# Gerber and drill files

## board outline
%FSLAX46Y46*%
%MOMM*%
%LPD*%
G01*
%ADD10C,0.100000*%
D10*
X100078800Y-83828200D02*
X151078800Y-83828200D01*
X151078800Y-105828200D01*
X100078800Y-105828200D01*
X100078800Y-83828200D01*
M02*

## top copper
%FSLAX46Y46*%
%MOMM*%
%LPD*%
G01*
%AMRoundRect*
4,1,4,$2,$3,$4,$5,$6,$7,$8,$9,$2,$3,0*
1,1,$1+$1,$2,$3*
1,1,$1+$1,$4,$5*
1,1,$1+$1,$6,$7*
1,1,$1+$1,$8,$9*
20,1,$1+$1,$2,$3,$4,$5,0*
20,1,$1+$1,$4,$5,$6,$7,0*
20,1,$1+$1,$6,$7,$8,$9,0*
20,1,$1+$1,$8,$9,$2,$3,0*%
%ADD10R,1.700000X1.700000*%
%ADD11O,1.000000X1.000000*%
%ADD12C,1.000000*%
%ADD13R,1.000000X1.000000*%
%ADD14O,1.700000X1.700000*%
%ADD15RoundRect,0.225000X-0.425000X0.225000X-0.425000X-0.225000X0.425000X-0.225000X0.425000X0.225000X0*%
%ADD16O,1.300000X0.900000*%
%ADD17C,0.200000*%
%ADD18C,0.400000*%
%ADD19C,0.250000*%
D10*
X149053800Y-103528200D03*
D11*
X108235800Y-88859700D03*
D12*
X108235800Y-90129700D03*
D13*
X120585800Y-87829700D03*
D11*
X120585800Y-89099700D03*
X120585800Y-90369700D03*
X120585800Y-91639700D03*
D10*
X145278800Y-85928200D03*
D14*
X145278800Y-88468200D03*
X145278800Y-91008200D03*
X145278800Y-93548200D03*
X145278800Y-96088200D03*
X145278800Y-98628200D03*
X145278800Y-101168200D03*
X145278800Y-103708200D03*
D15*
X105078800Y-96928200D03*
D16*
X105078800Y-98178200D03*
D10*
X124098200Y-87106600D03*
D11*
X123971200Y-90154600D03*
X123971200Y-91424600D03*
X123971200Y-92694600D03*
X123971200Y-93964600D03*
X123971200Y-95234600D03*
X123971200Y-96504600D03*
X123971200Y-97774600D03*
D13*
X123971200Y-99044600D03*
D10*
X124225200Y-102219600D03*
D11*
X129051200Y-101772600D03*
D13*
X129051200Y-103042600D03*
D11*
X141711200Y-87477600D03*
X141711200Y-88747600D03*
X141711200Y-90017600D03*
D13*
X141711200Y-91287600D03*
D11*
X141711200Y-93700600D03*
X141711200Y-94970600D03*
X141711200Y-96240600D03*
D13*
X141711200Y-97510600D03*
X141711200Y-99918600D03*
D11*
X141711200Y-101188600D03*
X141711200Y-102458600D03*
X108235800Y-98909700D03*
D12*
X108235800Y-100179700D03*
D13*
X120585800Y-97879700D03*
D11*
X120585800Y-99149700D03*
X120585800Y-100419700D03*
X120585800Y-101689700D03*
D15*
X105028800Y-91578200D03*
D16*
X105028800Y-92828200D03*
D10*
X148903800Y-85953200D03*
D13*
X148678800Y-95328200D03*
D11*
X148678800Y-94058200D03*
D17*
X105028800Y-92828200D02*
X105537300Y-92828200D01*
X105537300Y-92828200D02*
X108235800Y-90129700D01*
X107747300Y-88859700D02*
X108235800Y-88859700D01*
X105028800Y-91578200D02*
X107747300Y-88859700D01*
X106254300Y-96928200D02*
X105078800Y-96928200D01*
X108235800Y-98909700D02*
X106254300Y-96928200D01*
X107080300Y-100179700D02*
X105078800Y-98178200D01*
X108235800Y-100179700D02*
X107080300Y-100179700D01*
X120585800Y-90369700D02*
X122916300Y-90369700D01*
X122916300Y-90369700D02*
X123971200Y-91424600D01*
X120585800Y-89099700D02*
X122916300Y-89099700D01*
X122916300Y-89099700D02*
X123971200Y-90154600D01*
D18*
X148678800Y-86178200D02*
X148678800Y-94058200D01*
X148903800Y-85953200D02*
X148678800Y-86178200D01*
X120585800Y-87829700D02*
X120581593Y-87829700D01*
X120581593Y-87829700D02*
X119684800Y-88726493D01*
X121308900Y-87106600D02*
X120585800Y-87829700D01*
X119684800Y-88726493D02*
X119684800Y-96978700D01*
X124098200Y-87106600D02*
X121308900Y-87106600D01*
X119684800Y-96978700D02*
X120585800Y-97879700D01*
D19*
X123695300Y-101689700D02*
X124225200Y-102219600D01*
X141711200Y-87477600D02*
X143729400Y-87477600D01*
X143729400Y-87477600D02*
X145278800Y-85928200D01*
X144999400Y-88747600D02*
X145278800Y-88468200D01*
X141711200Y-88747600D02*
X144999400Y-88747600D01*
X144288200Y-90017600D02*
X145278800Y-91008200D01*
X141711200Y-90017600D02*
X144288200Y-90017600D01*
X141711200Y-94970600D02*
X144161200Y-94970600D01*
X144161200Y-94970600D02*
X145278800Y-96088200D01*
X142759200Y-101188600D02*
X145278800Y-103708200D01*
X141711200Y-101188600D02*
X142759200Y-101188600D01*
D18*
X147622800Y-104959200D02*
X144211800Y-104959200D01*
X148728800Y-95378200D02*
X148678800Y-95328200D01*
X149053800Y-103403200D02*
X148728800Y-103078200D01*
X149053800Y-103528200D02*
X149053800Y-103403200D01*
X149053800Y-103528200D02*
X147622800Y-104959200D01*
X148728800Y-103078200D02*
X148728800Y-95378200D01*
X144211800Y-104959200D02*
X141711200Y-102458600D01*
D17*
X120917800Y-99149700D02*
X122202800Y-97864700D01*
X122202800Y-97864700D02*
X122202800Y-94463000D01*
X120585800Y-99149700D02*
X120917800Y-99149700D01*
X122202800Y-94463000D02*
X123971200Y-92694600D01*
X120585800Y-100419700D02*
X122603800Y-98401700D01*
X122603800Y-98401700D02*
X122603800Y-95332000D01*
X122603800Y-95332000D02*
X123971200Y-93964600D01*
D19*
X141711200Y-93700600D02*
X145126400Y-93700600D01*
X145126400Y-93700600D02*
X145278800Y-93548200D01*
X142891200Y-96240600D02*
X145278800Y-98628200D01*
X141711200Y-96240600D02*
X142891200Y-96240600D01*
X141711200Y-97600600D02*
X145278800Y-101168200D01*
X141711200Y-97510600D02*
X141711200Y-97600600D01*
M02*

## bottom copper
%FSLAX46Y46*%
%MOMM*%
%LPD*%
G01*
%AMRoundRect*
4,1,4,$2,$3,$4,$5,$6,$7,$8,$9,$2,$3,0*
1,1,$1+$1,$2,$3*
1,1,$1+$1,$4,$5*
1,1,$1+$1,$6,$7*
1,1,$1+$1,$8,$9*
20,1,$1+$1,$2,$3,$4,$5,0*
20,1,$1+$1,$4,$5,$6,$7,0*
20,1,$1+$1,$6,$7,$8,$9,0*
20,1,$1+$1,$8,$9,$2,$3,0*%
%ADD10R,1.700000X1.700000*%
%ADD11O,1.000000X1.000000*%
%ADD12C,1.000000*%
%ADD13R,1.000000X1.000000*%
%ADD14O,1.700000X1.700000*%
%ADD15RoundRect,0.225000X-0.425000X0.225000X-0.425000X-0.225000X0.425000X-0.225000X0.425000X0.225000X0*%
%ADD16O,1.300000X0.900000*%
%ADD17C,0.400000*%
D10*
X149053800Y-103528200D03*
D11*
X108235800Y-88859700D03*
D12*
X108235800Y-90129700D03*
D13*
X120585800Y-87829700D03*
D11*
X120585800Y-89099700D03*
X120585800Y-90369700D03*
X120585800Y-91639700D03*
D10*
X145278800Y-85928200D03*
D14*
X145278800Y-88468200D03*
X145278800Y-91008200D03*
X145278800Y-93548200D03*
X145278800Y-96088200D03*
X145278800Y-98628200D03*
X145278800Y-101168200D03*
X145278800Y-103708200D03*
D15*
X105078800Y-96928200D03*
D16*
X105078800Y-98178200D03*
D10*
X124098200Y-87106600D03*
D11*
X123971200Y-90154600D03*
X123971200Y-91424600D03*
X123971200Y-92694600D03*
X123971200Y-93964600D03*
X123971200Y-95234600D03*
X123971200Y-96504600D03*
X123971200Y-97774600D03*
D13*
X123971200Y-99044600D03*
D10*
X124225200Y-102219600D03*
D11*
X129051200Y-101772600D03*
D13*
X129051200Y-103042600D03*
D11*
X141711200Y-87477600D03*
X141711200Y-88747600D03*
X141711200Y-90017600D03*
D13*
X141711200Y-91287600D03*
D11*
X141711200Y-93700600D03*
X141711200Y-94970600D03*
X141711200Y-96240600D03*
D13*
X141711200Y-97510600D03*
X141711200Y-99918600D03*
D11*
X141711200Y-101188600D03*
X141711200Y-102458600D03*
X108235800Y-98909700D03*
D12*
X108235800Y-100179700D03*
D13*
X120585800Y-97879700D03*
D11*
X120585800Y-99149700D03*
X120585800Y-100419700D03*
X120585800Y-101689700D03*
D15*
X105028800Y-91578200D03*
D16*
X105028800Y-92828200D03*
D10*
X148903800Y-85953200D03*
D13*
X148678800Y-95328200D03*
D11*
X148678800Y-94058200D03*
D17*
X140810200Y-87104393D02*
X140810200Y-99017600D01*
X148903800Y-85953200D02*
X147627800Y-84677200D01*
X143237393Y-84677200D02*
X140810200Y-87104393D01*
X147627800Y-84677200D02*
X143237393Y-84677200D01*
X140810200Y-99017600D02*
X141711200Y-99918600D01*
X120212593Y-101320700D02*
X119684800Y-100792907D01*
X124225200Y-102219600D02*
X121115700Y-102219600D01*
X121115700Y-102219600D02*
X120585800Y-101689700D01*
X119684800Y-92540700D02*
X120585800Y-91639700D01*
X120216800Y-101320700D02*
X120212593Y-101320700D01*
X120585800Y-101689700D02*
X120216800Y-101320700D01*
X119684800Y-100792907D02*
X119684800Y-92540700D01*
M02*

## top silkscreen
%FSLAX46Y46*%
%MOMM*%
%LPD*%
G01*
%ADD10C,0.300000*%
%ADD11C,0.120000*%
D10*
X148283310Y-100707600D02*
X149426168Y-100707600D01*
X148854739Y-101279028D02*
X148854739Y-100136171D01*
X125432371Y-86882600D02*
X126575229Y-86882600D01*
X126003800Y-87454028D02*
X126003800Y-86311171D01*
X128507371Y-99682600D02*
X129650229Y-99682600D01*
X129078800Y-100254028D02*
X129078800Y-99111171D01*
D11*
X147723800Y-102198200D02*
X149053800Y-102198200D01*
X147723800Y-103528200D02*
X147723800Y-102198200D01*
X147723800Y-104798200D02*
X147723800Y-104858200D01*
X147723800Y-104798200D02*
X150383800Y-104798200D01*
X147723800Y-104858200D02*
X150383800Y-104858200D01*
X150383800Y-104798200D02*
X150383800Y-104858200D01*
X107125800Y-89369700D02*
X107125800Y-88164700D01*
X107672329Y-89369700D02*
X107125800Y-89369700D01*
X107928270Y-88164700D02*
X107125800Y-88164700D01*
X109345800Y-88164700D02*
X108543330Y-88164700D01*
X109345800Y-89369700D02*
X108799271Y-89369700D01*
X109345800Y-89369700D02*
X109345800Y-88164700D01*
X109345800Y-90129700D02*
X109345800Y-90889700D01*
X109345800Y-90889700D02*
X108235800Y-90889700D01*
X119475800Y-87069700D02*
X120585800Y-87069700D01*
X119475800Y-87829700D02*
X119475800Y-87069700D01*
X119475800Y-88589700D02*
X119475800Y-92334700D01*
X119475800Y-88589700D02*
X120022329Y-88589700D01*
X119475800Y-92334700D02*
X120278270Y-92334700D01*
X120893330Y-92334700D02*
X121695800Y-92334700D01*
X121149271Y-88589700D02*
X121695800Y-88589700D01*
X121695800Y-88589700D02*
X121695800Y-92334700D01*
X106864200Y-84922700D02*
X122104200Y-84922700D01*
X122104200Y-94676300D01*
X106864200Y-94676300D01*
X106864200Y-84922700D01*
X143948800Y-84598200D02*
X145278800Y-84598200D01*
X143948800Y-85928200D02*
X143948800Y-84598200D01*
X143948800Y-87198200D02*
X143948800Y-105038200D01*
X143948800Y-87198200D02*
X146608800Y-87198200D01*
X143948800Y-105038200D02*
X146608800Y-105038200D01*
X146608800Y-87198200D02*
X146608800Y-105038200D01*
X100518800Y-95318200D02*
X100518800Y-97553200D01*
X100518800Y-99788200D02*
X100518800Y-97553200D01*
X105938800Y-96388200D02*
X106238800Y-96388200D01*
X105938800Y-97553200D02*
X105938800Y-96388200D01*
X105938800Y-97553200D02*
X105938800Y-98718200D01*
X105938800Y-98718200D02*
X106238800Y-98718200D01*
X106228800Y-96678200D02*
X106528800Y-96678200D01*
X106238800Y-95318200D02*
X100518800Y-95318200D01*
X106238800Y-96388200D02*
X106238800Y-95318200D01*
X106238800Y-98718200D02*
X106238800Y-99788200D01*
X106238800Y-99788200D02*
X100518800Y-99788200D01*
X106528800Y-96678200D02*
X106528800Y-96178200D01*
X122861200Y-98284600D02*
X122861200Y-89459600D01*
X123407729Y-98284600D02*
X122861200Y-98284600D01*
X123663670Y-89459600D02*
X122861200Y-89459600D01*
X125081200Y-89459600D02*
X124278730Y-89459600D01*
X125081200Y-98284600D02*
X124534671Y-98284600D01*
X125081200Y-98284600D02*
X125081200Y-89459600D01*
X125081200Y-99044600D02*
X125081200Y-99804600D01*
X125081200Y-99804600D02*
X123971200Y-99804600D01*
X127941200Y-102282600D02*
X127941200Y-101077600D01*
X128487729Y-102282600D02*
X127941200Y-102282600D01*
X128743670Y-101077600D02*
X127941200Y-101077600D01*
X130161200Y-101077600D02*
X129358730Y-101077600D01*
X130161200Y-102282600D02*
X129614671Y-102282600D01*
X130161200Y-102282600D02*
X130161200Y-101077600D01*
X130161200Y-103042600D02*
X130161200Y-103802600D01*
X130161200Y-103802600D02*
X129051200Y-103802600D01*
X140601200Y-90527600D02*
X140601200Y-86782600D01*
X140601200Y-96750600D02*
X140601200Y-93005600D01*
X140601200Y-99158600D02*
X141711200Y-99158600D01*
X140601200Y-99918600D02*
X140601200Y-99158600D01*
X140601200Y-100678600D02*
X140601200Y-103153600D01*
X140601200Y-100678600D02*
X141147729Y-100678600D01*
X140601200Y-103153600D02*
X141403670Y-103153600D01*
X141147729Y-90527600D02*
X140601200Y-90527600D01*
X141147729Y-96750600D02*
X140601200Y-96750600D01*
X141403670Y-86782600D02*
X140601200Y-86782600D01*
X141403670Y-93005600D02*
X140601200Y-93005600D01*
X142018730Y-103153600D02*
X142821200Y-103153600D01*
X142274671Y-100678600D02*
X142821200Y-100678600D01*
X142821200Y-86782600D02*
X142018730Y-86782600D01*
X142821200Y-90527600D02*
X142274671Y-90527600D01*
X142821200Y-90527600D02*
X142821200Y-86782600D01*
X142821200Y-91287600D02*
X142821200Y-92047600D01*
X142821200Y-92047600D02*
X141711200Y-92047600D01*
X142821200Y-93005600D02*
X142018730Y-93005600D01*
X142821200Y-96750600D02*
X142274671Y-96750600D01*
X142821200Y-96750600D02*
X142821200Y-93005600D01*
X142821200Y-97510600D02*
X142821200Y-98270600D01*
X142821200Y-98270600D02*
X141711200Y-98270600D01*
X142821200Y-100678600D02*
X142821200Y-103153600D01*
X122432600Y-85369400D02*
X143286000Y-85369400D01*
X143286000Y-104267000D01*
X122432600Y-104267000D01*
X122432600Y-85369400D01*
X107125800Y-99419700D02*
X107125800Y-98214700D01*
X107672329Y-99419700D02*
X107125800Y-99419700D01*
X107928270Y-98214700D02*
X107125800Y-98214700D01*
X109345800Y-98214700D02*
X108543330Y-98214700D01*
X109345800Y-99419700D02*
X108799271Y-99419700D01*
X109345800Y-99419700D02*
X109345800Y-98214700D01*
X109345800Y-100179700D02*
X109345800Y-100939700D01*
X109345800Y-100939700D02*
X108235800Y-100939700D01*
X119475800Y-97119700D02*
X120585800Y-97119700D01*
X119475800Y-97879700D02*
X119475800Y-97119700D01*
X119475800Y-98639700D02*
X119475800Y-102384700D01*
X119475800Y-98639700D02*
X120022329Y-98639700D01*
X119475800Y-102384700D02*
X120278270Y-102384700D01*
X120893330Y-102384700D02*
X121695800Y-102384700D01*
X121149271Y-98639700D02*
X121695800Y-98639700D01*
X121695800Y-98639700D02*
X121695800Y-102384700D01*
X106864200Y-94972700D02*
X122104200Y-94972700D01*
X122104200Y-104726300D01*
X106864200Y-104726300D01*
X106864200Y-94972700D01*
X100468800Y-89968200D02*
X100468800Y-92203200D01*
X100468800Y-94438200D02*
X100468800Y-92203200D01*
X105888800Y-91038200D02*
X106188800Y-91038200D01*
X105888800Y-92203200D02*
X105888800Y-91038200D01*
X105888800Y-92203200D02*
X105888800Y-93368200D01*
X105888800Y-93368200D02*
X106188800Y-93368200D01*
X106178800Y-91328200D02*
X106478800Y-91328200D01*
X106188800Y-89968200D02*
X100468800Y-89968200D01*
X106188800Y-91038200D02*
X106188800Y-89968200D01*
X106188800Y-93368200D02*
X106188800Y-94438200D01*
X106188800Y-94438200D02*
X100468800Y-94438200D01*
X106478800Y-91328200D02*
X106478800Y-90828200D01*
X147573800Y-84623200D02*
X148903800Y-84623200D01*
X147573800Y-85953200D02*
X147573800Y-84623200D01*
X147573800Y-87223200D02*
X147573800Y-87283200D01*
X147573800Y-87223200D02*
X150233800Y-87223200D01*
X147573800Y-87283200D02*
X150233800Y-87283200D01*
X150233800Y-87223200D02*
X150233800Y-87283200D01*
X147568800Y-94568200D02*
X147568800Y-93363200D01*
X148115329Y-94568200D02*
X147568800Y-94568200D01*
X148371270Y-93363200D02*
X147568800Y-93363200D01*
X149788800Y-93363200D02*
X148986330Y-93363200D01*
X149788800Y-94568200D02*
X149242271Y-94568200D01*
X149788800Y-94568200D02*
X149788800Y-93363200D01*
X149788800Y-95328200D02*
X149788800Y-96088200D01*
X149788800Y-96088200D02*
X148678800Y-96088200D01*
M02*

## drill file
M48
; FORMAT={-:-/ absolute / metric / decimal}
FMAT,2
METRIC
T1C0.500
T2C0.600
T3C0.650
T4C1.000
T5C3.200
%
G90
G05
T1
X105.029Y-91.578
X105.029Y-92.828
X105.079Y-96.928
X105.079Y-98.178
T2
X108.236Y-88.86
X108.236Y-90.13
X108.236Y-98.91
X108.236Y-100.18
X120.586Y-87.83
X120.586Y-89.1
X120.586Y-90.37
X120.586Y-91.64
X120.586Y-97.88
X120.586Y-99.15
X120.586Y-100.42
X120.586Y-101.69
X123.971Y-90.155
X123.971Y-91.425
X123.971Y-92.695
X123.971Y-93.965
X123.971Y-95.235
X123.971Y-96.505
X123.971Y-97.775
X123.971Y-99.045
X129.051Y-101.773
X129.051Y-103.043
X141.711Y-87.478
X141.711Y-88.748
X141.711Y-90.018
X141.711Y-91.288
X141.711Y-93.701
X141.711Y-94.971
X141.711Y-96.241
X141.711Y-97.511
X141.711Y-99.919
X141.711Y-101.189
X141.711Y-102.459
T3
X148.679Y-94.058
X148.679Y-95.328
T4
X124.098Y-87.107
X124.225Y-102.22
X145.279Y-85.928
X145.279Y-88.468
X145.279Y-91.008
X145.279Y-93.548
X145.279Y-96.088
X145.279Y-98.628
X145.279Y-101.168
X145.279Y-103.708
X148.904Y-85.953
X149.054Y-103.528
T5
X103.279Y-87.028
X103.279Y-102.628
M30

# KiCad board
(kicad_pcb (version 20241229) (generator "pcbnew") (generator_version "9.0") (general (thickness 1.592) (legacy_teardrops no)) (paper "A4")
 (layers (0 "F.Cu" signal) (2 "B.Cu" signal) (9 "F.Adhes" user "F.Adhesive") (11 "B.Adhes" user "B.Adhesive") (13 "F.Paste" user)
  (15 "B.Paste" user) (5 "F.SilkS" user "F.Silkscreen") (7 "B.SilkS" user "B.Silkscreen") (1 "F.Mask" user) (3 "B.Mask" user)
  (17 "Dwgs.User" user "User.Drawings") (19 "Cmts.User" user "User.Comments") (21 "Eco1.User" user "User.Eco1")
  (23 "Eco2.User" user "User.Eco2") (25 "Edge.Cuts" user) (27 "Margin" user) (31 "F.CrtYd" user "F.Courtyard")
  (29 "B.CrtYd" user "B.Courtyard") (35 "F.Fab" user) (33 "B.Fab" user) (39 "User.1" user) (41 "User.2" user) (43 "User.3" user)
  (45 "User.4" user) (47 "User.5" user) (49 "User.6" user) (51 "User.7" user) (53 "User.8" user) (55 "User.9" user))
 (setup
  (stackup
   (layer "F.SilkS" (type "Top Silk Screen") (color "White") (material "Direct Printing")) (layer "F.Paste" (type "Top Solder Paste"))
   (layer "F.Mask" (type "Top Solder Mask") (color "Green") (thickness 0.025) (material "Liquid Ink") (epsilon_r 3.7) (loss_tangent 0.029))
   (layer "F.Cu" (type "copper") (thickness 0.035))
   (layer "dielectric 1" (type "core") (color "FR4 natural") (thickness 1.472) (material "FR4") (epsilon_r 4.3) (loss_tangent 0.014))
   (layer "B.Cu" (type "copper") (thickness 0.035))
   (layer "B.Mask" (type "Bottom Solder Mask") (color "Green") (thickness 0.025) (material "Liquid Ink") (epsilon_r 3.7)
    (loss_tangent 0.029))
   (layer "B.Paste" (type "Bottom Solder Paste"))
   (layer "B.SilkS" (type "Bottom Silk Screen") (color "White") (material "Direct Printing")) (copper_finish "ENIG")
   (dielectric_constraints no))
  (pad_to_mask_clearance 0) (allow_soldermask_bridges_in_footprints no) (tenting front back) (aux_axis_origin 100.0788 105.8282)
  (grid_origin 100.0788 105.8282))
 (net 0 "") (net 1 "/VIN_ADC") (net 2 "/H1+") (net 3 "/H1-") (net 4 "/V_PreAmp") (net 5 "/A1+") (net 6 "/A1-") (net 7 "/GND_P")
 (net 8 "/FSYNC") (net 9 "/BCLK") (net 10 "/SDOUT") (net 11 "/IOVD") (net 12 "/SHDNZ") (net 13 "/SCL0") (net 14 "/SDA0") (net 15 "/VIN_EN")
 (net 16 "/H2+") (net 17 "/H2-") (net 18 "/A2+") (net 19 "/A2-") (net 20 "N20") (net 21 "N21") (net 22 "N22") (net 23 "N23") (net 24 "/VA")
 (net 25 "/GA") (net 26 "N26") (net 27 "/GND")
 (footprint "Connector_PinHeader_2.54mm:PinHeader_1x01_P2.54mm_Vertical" (layer "F.Cu") (at 149.0538 103.5282)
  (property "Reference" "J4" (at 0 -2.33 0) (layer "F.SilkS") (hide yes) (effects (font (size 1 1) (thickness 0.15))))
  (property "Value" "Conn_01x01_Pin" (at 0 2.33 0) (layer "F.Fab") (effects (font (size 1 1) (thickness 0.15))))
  (fp_line (start -1.33 -1.33) (end 0 -1.33) (stroke (width 0.12) (type solid)) (layer "F.SilkS"))
  (fp_line (start -1.33 0) (end -1.33 -1.33) (stroke (width 0.12) (type solid)) (layer "F.SilkS"))
  (fp_line (start -1.33 1.27) (end -1.33 1.33) (stroke (width 0.12) (type solid)) (layer "F.SilkS"))
  (fp_line (start -1.33 1.27) (end 1.33 1.27) (stroke (width 0.12) (type solid)) (layer "F.SilkS"))
  (fp_line (start -1.33 1.33) (end 1.33 1.33) (stroke (width 0.12) (type solid)) (layer "F.SilkS"))
  (fp_line (start 1.33 1.27) (end 1.33 1.33) (stroke (width 0.12) (type solid)) (layer "F.SilkS"))
  (pad "1" thru_hole rect (at 0 0) (size 1.7 1.7) (drill 1) (layers "*.Cu" "*.Mask") (remove_unused_layers no) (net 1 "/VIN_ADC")))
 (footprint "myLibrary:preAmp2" (layer "F.Cu") (at 113.7222 89.3931)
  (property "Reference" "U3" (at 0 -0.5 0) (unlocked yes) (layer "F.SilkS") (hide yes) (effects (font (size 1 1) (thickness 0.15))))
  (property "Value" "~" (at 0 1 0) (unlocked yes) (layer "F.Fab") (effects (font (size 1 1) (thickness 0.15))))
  (fp_line (start -6.5964 -0.0234) (end -6.5964 -1.2284) (stroke (width 0.12) (type solid)) (layer "F.SilkS"))
  (fp_line (start -6.049871 -0.0234) (end -6.5964 -0.0234) (stroke (width 0.12) (type solid)) (layer "F.SilkS"))
  (fp_line (start -5.79393 -1.2284) (end -6.5964 -1.2284) (stroke (width 0.12) (type solid)) (layer "F.SilkS"))
  (fp_line (start -4.3764 -1.2284) (end -5.17887 -1.2284) (stroke (width 0.12) (type solid)) (layer "F.SilkS"))
  (fp_line (start -4.3764 -0.0234) (end -4.922929 -0.0234) (stroke (width 0.12) (type solid)) (layer "F.SilkS"))
  (fp_line (start -4.3764 -0.0234) (end -4.3764 -1.2284) (stroke (width 0.12) (type solid)) (layer "F.SilkS"))
  (fp_line (start -4.3764 0.7366) (end -4.3764 1.4966) (stroke (width 0.12) (type solid)) (layer "F.SilkS"))
  (fp_line (start -4.3764 1.4966) (end -5.4864 1.4966) (stroke (width 0.12) (type solid)) (layer "F.SilkS"))
  (fp_line (start 5.7536 -2.3234) (end 6.8636 -2.3234) (stroke (width 0.12) (type solid)) (layer "F.SilkS"))
  (fp_line (start 5.7536 -1.5634) (end 5.7536 -2.3234) (stroke (width 0.12) (type solid)) (layer "F.SilkS"))
  (fp_line (start 5.7536 -0.8034) (end 5.7536 2.9416) (stroke (width 0.12) (type solid)) (layer "F.SilkS"))
  (fp_line (start 5.7536 -0.8034) (end 6.300129 -0.8034) (stroke (width 0.12) (type solid)) (layer "F.SilkS"))
  (fp_line (start 5.7536 2.9416) (end 6.55607 2.9416) (stroke (width 0.12) (type solid)) (layer "F.SilkS"))
  (fp_line (start 7.17113 2.9416) (end 7.9736 2.9416) (stroke (width 0.12) (type solid)) (layer "F.SilkS"))
  (fp_line (start 7.427071 -0.8034) (end 7.9736 -0.8034) (stroke (width 0.12) (type solid)) (layer "F.SilkS"))
  (fp_line (start 7.9736 -0.8034) (end 7.9736 2.9416) (stroke (width 0.12) (type solid)) (layer "F.SilkS"))
  (fp_rect (start -6.858 -4.4704) (end 8.382 5.2832) (stroke (width 0.12) (type default)) (fill no) (layer "F.SilkS"))
  (pad "1" thru_hole oval (at -5.4864 -0.5334 180) (size 1 1) (drill 0.6) (layers "*.Cu" "*.Mask") (remove_unused_layers no) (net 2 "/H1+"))
  (pad "2" thru_hole circle (at -5.4864 0.7366 180) (size 1 1) (drill 0.6) (layers "*.Cu" "*.Mask") (remove_unused_layers no) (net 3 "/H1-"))
  (pad "3" thru_hole rect (at 6.8636 -1.5634) (size 1 1) (drill 0.6) (layers "*.Cu" "*.Mask") (remove_unused_layers no) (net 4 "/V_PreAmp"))
  (pad "4" thru_hole oval (at 6.8636 -0.2934) (size 1 1) (drill 0.6) (layers "*.Cu" "*.Mask") (remove_unused_layers no) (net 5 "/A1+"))
  (pad "5" thru_hole oval (at 6.8636 0.9766) (size 1 1) (drill 0.6) (layers "*.Cu" "*.Mask") (remove_unused_layers no) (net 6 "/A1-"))
  (pad "6" thru_hole oval (at 6.8636 2.2466) (size 1 1) (drill 0.6) (layers "*.Cu" "*.Mask") (remove_unused_layers no) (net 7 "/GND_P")))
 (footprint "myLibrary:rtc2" (layer "F.Cu") (at 212.5538 102.4732 180)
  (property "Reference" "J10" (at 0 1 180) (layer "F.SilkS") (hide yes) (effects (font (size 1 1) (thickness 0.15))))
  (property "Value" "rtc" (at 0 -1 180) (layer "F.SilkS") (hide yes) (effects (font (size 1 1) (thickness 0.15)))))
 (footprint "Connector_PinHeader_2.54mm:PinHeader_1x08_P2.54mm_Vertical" (layer "F.Cu") (at 145.2788 85.9282)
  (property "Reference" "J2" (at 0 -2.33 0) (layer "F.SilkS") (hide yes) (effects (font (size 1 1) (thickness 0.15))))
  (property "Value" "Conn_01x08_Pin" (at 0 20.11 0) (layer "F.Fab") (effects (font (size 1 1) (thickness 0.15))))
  (fp_line (start -1.33 -1.33) (end 0 -1.33) (stroke (width 0.12) (type solid)) (layer "F.SilkS"))
  (fp_line (start -1.33 0) (end -1.33 -1.33) (stroke (width 0.12) (type solid)) (layer "F.SilkS"))
  (fp_line (start -1.33 1.27) (end -1.33 19.11) (stroke (width 0.12) (type solid)) (layer "F.SilkS"))
  (fp_line (start -1.33 1.27) (end 1.33 1.27) (stroke (width 0.12) (type solid)) (layer "F.SilkS"))
  (fp_line (start -1.33 19.11) (end 1.33 19.11) (stroke (width 0.12) (type solid)) (layer "F.SilkS"))
  (fp_line (start 1.33 1.27) (end 1.33 19.11) (stroke (width 0.12) (type solid)) (layer "F.SilkS"))
  (pad "1" thru_hole rect (at 0 0) (size 1.7 1.7) (drill 1) (layers "*.Cu" "*.Mask") (remove_unused_layers no) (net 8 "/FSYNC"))
  (pad "2" thru_hole oval (at 0 2.54) (size 1.7 1.7) (drill 1) (layers "*.Cu" "*.Mask") (remove_unused_layers no) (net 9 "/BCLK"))
  (pad "3" thru_hole oval (at 0 5.08) (size 1.7 1.7) (drill 1) (layers "*.Cu" "*.Mask") (remove_unused_layers no) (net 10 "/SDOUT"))
  (pad "4" thru_hole oval (at 0 7.62) (size 1.7 1.7) (drill 1) (layers "*.Cu" "*.Mask") (remove_unused_layers no) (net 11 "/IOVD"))
  (pad "5" thru_hole oval (at 0 10.16) (size 1.7 1.7) (drill 1) (layers "*.Cu" "*.Mask") (remove_unused_layers no) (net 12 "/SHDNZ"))
  (pad "6" thru_hole oval (at 0 12.7) (size 1.7 1.7) (drill 1) (layers "*.Cu" "*.Mask") (remove_unused_layers no) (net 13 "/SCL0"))
  (pad "7" thru_hole oval (at 0 15.24) (size 1.7 1.7) (drill 1) (layers "*.Cu" "*.Mask") (remove_unused_layers no) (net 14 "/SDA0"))
  (pad "8" thru_hole oval (at 0 17.78) (size 1.7 1.7) (drill 1) (layers "*.Cu" "*.Mask") (remove_unused_layers no) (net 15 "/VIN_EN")))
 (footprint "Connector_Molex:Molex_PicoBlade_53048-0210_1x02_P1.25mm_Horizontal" (layer "F.Cu") (at 105.0788 96.9282 -90)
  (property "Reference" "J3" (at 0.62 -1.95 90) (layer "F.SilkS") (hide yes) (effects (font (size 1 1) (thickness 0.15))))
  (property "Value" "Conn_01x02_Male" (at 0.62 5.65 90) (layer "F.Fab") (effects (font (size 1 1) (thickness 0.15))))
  (fp_line (start -1.61 4.56) (end 0.625 4.56) (stroke (width 0.12) (type solid)) (layer "F.SilkS"))
  (fp_line (start 2.86 4.56) (end 0.625 4.56) (stroke (width 0.12) (type solid)) (layer "F.SilkS"))
  (fp_line (start -0.54 -0.86) (end -0.54 -1.16) (stroke (width 0.12) (type solid)) (layer "F.SilkS"))
  (fp_line (start 0.625 -0.86) (end -0.54 -0.86) (stroke (width 0.12) (type solid)) (layer "F.SilkS"))
  (fp_line (start 0.625 -0.86) (end 1.79 -0.86) (stroke (width 0.12) (type solid)) (layer "F.SilkS"))
  (fp_line (start 1.79 -0.86) (end 1.79 -1.16) (stroke (width 0.12) (type solid)) (layer "F.SilkS"))
  (fp_line (start -0.25 -1.15) (end -0.25 -1.45) (stroke (width 0.12) (type solid)) (layer "F.SilkS"))
  (fp_line (start -1.61 -1.16) (end -1.61 4.56) (stroke (width 0.12) (type solid)) (layer "F.SilkS"))
  (fp_line (start -0.54 -1.16) (end -1.61 -1.16) (stroke (width 0.12) (type solid)) (layer "F.SilkS"))
  (fp_line (start 1.79 -1.16) (end 2.86 -1.16) (stroke (width 0.12) (type solid)) (layer "F.SilkS"))
  (fp_line (start 2.86 -1.16) (end 2.86 4.56) (stroke (width 0.12) (type solid)) (layer "F.SilkS"))
  (fp_line (start -0.25 -1.45) (end -0.75 -1.45) (stroke (width 0.12) (type solid)) (layer "F.SilkS"))
  (pad "1" thru_hole roundrect (at 0 0 270) (size 0.9 1.3) (drill 0.5) (layers "*.Cu" "*.Mask") (remove_unused_layers no)
   (roundrect_rratio 0.25) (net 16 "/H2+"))
  (pad "2" thru_hole oval (at 1.25 0 270) (size 0.9 1.3) (drill 0.5) (layers "*.Cu" "*.Mask") (remove_unused_layers no) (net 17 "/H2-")))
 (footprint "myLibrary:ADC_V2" (layer "F.Cu") (at 133.3038 95.4532)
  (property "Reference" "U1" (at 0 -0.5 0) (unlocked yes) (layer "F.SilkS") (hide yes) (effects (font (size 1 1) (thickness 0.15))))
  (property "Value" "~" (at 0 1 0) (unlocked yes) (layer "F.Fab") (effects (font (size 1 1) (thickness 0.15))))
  (fp_line (start -10.4426 2.8314) (end -10.4426 -5.9936) (stroke (width 0.12) (type solid)) (layer "F.SilkS"))
  (fp_line (start -9.896071 2.8314) (end -10.4426 2.8314) (stroke (width 0.12) (type solid)) (layer "F.SilkS"))
  (fp_line (start -9.64013 -5.9936) (end -10.4426 -5.9936) (stroke (width 0.12) (type solid)) (layer "F.SilkS"))
  (fp_line (start -8.2226 -5.9936) (end -9.02507 -5.9936) (stroke (width 0.12) (type solid)) (layer "F.SilkS"))
  (fp_line (start -8.2226 2.8314) (end -8.769129 2.8314) (stroke (width 0.12) (type solid)) (layer "F.SilkS"))
  (fp_line (start -8.2226 2.8314) (end -8.2226 -5.9936) (stroke (width 0.12) (type solid)) (layer "F.SilkS"))
  (fp_line (start -8.2226 3.5914) (end -8.2226 4.3514) (stroke (width 0.12) (type solid)) (layer "F.SilkS"))
  (fp_line (start -8.2226 4.3514) (end -9.3326 4.3514) (stroke (width 0.12) (type solid)) (layer "F.SilkS"))
  (fp_line (start -5.3626 6.8294) (end -5.3626 5.6244) (stroke (width 0.12) (type solid)) (layer "F.SilkS"))
  (fp_line (start -4.816071 6.8294) (end -5.3626 6.8294) (stroke (width 0.12) (type solid)) (layer "F.SilkS"))
  (fp_line (start -4.56013 5.6244) (end -5.3626 5.6244) (stroke (width 0.12) (type solid)) (layer "F.SilkS"))
  (fp_line (start -3.1426 5.6244) (end -3.94507 5.6244) (stroke (width 0.12) (type solid)) (layer "F.SilkS"))
  (fp_line (start -3.1426 6.8294) (end -3.689129 6.8294) (stroke (width 0.12) (type solid)) (layer "F.SilkS"))
  (fp_line (start -3.1426 6.8294) (end -3.1426 5.6244) (stroke (width 0.12) (type solid)) (layer "F.SilkS"))
  (fp_line (start -3.1426 7.5894) (end -3.1426 8.3494) (stroke (width 0.12) (type solid)) (layer "F.SilkS"))
  (fp_line (start -3.1426 8.3494) (end -4.2526 8.3494) (stroke (width 0.12) (type solid)) (layer "F.SilkS"))
  (fp_line (start 7.2974 -4.9256) (end 7.2974 -8.6706) (stroke (width 0.12) (type solid)) (layer "F.SilkS"))
  (fp_line (start 7.2974 1.2974) (end 7.2974 -2.4476) (stroke (width 0.12) (type solid)) (layer "F.SilkS"))
  (fp_line (start 7.2974 3.7054) (end 8.4074 3.7054) (stroke (width 0.12) (type solid)) (layer "F.SilkS"))
  (fp_line (start 7.2974 4.4654) (end 7.2974 3.7054) (stroke (width 0.12) (type solid)) (layer "F.SilkS"))
  (fp_line (start 7.2974 5.2254) (end 7.2974 7.7004) (stroke (width 0.12) (type solid)) (layer "F.SilkS"))
  (fp_line (start 7.2974 5.2254) (end 7.843929 5.2254) (stroke (width 0.12) (type solid)) (layer "F.SilkS"))
  (fp_line (start 7.2974 7.7004) (end 8.09987 7.7004) (stroke (width 0.12) (type solid)) (layer "F.SilkS"))
  (fp_line (start 7.843929 -4.9256) (end 7.2974 -4.9256) (stroke (width 0.12) (type solid)) (layer "F.SilkS"))
  (fp_line (start 7.843929 1.2974) (end 7.2974 1.2974) (stroke (width 0.12) (type solid)) (layer "F.SilkS"))
  (fp_line (start 8.09987 -8.6706) (end 7.2974 -8.6706) (stroke (width 0.12) (type solid)) (layer "F.SilkS"))
  (fp_line (start 8.09987 -2.4476) (end 7.2974 -2.4476) (stroke (width 0.12) (type solid)) (layer "F.SilkS"))
  (fp_line (start 8.71493 7.7004) (end 9.5174 7.7004) (stroke (width 0.12) (type solid)) (layer "F.SilkS"))
  (fp_line (start 8.970871 5.2254) (end 9.5174 5.2254) (stroke (width 0.12) (type solid)) (layer "F.SilkS"))
  (fp_line (start 9.5174 -8.6706) (end 8.71493 -8.6706) (stroke (width 0.12) (type solid)) (layer "F.SilkS"))
  (fp_line (start 9.5174 -4.9256) (end 8.970871 -4.9256) (stroke (width 0.12) (type solid)) (layer "F.SilkS"))
  (fp_line (start 9.5174 -4.9256) (end 9.5174 -8.6706) (stroke (width 0.12) (type solid)) (layer "F.SilkS"))
  (fp_line (start 9.5174 -4.1656) (end 9.5174 -3.4056) (stroke (width 0.12) (type solid)) (layer "F.SilkS"))
  (fp_line (start 9.5174 -3.4056) (end 8.4074 -3.4056) (stroke (width 0.12) (type solid)) (layer "F.SilkS"))
  (fp_line (start 9.5174 -2.4476) (end 8.71493 -2.4476) (stroke (width 0.12) (type solid)) (layer "F.SilkS"))
  (fp_line (start 9.5174 1.2974) (end 8.970871 1.2974) (stroke (width 0.12) (type solid)) (layer "F.SilkS"))
  (fp_line (start 9.5174 1.2974) (end 9.5174 -2.4476) (stroke (width 0.12) (type solid)) (layer "F.SilkS"))
  (fp_line (start 9.5174 2.0574) (end 9.5174 2.8174) (stroke (width 0.12) (type solid)) (layer "F.SilkS"))
  (fp_line (start 9.5174 2.8174) (end 8.4074 2.8174) (stroke (width 0.12) (type solid)) (layer "F.SilkS"))
  (fp_line (start 9.5174 5.2254) (end 9.5174 7.7004) (stroke (width 0.12) (type solid)) (layer "F.SilkS"))
  (fp_rect (start -10.8712 -10.0838) (end 9.9822 8.8138) (stroke (width 0.12) (type default)) (fill no) (layer "F.SilkS"))
  (pad "1" thru_hole rect (at -9.2056 -8.3466) (size 1.7 1.7) (drill 1) (layers "*.Cu" "*.Mask") (remove_unused_layers no)
   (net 4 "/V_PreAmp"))
  (pad "2" thru_hole oval (at -9.3326 -5.2986 180) (size 1 1) (drill 0.6) (layers "*.Cu" "*.Mask") (remove_unused_layers no) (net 5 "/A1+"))
  (pad "3" thru_hole oval (at -9.3326 -4.0286 180) (size 1 1) (drill 0.6) (layers "*.Cu" "*.Mask") (remove_unused_layers no) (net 6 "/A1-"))
  (pad "4" thru_hole oval (at -9.3326 -2.7586 180) (size 1 1) (drill 0.6) (layers "*.Cu" "*.Mask") (remove_unused_layers no) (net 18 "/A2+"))
  (pad "5" thru_hole oval (at -9.3326 -1.4886 180) (size 1 1) (drill 0.6) (layers "*.Cu" "*.Mask") (remove_unused_layers no) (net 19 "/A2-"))
  (pad "6" thru_hole oval (at -9.3326 -0.2186 180) (size 1 1) (drill 0.6) (layers "*.Cu" "*.Mask") (remove_unused_layers no) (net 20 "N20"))
  (pad "7" thru_hole oval (at -9.3326 1.0514 180) (size 1 1) (drill 0.6) (layers "*.Cu" "*.Mask") (remove_unused_layers no) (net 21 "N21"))
  (pad "8" thru_hole oval (at -9.3326 2.3214 180) (size 1 1) (drill 0.6) (layers "*.Cu" "*.Mask") (remove_unused_layers no) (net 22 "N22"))
  (pad "9" thru_hole rect (at -9.3326 3.5914 180) (size 1 1) (drill 0.6) (layers "*.Cu" "*.Mask") (remove_unused_layers no) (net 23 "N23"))
  (pad "10" thru_hole rect (at -9.0786 6.7664) (size 1.7 1.7) (drill 1) (layers "*.Cu" "*.Mask") (remove_unused_layers no) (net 7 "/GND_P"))
  (pad "11" thru_hole oval (at -4.2526 6.3194 180) (size 1 1) (drill 0.6) (layers "*.Cu" "*.Mask") (remove_unused_layers no) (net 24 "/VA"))
  (pad "12" thru_hole rect (at -4.2526 7.5894 180) (size 1 1) (drill 0.6) (layers "*.Cu" "*.Mask") (remove_unused_layers no) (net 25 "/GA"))
  (pad "13" thru_hole oval (at 8.4074 -7.9756 180) (size 1 1) (drill 0.6) (layers "*.Cu" "*.Mask") (remove_unused_layers no)
   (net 8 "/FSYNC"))
  (pad "14" thru_hole oval (at 8.4074 -6.7056 180) (size 1 1) (drill 0.6) (layers "*.Cu" "*.Mask") (remove_unused_layers no) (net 9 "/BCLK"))
  (pad "15" thru_hole oval (at 8.4074 -5.4356 180) (size 1 1) (drill 0.6) (layers "*.Cu" "*.Mask") (remove_unused_layers no)
   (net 10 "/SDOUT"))
  (pad "16" thru_hole rect (at 8.4074 -4.1656 180) (size 1 1) (drill 0.6) (layers "*.Cu" "*.Mask") (remove_unused_layers no) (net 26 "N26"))
  (pad "17" thru_hole oval (at 8.4074 -1.7526 180) (size 1 1) (drill 0.6) (layers "*.Cu" "*.Mask") (remove_unused_layers no)
   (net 11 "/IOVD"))
  (pad "18" thru_hole oval (at 8.4074 -0.4826 180) (size 1 1) (drill 0.6) (layers "*.Cu" "*.Mask") (remove_unused_layers no)
   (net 12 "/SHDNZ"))
  (pad "19" thru_hole oval (at 8.4074 0.7874 180) (size 1 1) (drill 0.6) (layers "*.Cu" "*.Mask") (remove_unused_layers no) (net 13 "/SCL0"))
  (pad "20" thru_hole rect (at 8.4074 2.0574 180) (size 1 1) (drill 0.6) (layers "*.Cu" "*.Mask") (remove_unused_layers no) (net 14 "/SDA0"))
  (pad "21" thru_hole rect (at 8.4074 4.4654) (size 1 1) (drill 0.6) (layers "*.Cu" "*.Mask") (remove_unused_layers no) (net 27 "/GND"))
  (pad "22" thru_hole oval (at 8.4074 5.7354) (size 1 1) (drill 0.6) (layers "*.Cu" "*.Mask") (remove_unused_layers no) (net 15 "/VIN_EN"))
  (pad "23" thru_hole oval (at 8.4074 7.0054) (size 1 1) (drill 0.6) (layers "*.Cu" "*.Mask") (remove_unused_layers no) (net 1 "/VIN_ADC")))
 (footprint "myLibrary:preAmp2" (layer "F.Cu") (at 113.7222 99.4431)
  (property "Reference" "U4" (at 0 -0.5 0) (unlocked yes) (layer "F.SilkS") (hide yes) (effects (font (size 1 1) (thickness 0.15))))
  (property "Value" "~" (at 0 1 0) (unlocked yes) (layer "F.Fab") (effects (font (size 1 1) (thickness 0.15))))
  (fp_line (start -6.5964 -0.0234) (end -6.5964 -1.2284) (stroke (width 0.12) (type solid)) (layer "F.SilkS"))
  (fp_line (start -6.049871 -0.0234) (end -6.5964 -0.0234) (stroke (width 0.12) (type solid)) (layer "F.SilkS"))
  (fp_line (start -5.79393 -1.2284) (end -6.5964 -1.2284) (stroke (width 0.12) (type solid)) (layer "F.SilkS"))
  (fp_line (start -4.3764 -1.2284) (end -5.17887 -1.2284) (stroke (width 0.12) (type solid)) (layer "F.SilkS"))
  (fp_line (start -4.3764 -0.0234) (end -4.922929 -0.0234) (stroke (width 0.12) (type solid)) (layer "F.SilkS"))
  (fp_line (start -4.3764 -0.0234) (end -4.3764 -1.2284) (stroke (width 0.12) (type solid)) (layer "F.SilkS"))
  (fp_line (start -4.3764 0.7366) (end -4.3764 1.4966) (stroke (width 0.12) (type solid)) (layer "F.SilkS"))
  (fp_line (start -4.3764 1.4966) (end -5.4864 1.4966) (stroke (width 0.12) (type solid)) (layer "F.SilkS"))
  (fp_line (start 5.7536 -2.3234) (end 6.8636 -2.3234) (stroke (width 0.12) (type solid)) (layer "F.SilkS"))
  (fp_line (start 5.7536 -1.5634) (end 5.7536 -2.3234) (stroke (width 0.12) (type solid)) (layer "F.SilkS"))
  (fp_line (start 5.7536 -0.8034) (end 5.7536 2.9416) (stroke (width 0.12) (type solid)) (layer "F.SilkS"))
  (fp_line (start 5.7536 -0.8034) (end 6.300129 -0.8034) (stroke (width 0.12) (type solid)) (layer "F.SilkS"))
  (fp_line (start 5.7536 2.9416) (end 6.55607 2.9416) (stroke (width 0.12) (type solid)) (layer "F.SilkS"))
  (fp_line (start 7.17113 2.9416) (end 7.9736 2.9416) (stroke (width 0.12) (type solid)) (layer "F.SilkS"))
  (fp_line (start 7.427071 -0.8034) (end 7.9736 -0.8034) (stroke (width 0.12) (type solid)) (layer "F.SilkS"))
  (fp_line (start 7.9736 -0.8034) (end 7.9736 2.9416) (stroke (width 0.12) (type solid)) (layer "F.SilkS"))
  (fp_rect (start -6.858 -4.4704) (end 8.382 5.2832) (stroke (width 0.12) (type default)) (fill no) (layer "F.SilkS"))
  (pad "1" thru_hole oval (at -5.4864 -0.5334 180) (size 1 1) (drill 0.6) (layers "*.Cu" "*.Mask") (remove_unused_layers no) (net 16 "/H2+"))
  (pad "2" thru_hole circle (at -5.4864 0.7366 180) (size 1 1) (drill 0.6) (layers "*.Cu" "*.Mask") (remove_unused_layers no)
   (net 17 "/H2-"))
  (pad "3" thru_hole rect (at 6.8636 -1.5634) (size 1 1) (drill 0.6) (layers "*.Cu" "*.Mask") (remove_unused_layers no) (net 4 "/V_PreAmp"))
  (pad "4" thru_hole oval (at 6.8636 -0.2934) (size 1 1) (drill 0.6) (layers "*.Cu" "*.Mask") (remove_unused_layers no) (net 18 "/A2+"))
  (pad "5" thru_hole oval (at 6.8636 0.9766) (size 1 1) (drill 0.6) (layers "*.Cu" "*.Mask") (remove_unused_layers no) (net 19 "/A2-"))
  (pad "6" thru_hole oval (at 6.8636 2.2466) (size 1 1) (drill 0.6) (layers "*.Cu" "*.Mask") (remove_unused_layers no) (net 7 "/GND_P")))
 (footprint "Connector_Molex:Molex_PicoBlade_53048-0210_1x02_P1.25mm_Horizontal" (layer "F.Cu") (at 105.0288 91.5782 -90)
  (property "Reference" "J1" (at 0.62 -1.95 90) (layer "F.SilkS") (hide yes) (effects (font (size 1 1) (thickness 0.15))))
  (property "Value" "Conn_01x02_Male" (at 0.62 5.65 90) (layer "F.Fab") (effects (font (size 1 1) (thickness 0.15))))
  (fp_line (start -1.61 4.56) (end 0.625 4.56) (stroke (width 0.12) (type solid)) (layer "F.SilkS"))
  (fp_line (start 2.86 4.56) (end 0.625 4.56) (stroke (width 0.12) (type solid)) (layer "F.SilkS"))
  (fp_line (start -0.54 -0.86) (end -0.54 -1.16) (stroke (width 0.12) (type solid)) (layer "F.SilkS"))
  (fp_line (start 0.625 -0.86) (end -0.54 -0.86) (stroke (width 0.12) (type solid)) (layer "F.SilkS"))
  (fp_line (start 0.625 -0.86) (end 1.79 -0.86) (stroke (width 0.12) (type solid)) (layer "F.SilkS"))
  (fp_line (start 1.79 -0.86) (end 1.79 -1.16) (stroke (width 0.12) (type solid)) (layer "F.SilkS"))
  (fp_line (start -0.25 -1.15) (end -0.25 -1.45) (stroke (width 0.12) (type solid)) (layer "F.SilkS"))
  (fp_line (start -1.61 -1.16) (end -1.61 4.56) (stroke (width 0.12) (type solid)) (layer "F.SilkS"))
  (fp_line (start -0.54 -1.16) (end -1.61 -1.16) (stroke (width 0.12) (type solid)) (layer "F.SilkS"))
  (fp_line (start 1.79 -1.16) (end 2.86 -1.16) (stroke (width 0.12) (type solid)) (layer "F.SilkS"))
  (fp_line (start 2.86 -1.16) (end 2.86 4.56) (stroke (width 0.12) (type solid)) (layer "F.SilkS"))
  (fp_line (start -0.25 -1.45) (end -0.75 -1.45) (stroke (width 0.12) (type solid)) (layer "F.SilkS"))
  (pad "1" thru_hole roundrect (at 0 0 270) (size 0.9 1.3) (drill 0.5) (layers "*.Cu" "*.Mask") (remove_unused_layers no)
   (roundrect_rratio 0.25) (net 2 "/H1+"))
  (pad "2" thru_hole oval (at 1.25 0 270) (size 0.9 1.3) (drill 0.5) (layers "*.Cu" "*.Mask") (remove_unused_layers no) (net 3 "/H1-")))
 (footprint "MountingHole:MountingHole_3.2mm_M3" (layer "F.Cu") (at 103.2788 87.0282)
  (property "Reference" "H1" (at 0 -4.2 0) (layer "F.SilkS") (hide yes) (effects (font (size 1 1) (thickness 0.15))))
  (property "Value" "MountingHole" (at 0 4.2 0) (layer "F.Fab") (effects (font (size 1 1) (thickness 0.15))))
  (pad "" np_thru_hole circle (at 0 0) (size 3.2 3.2) (drill 3.2) (layers "*.Cu" "*.Mask")))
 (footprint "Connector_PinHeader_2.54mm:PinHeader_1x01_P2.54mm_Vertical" (layer "F.Cu") (at 148.9038 85.9532)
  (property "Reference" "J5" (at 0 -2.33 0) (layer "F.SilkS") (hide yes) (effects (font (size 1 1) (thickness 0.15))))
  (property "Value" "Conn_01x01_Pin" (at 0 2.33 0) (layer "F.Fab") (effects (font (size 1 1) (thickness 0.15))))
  (fp_line (start -1.33 -1.33) (end 0 -1.33) (stroke (width 0.12) (type solid)) (layer "F.SilkS"))
  (fp_line (start -1.33 0) (end -1.33 -1.33) (stroke (width 0.12) (type solid)) (layer "F.SilkS"))
  (fp_line (start -1.33 1.27) (end -1.33 1.33) (stroke (width 0.12) (type solid)) (layer "F.SilkS"))
  (fp_line (start -1.33 1.27) (end 1.33 1.27) (stroke (width 0.12) (type solid)) (layer "F.SilkS"))
  (fp_line (start -1.33 1.33) (end 1.33 1.33) (stroke (width 0.12) (type solid)) (layer "F.SilkS"))
  (fp_line (start 1.33 1.27) (end 1.33 1.33) (stroke (width 0.12) (type solid)) (layer "F.SilkS"))
  (pad "1" thru_hole rect (at 0 0) (size 1.7 1.7) (drill 1) (layers "*.Cu" "*.Mask") (remove_unused_layers no) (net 27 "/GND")))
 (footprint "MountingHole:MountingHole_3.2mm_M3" (layer "F.Cu") (at 103.2788 102.6282)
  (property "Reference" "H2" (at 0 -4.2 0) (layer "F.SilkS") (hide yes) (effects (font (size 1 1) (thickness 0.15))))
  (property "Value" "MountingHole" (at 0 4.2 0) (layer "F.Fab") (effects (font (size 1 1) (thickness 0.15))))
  (pad "" np_thru_hole circle (at 0 0) (size 3.2 3.2) (drill 3.2) (layers "*.Cu" "*.Mask")))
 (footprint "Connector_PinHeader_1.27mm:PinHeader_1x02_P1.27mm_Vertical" (layer "F.Cu") (at 148.6788 95.3282 180)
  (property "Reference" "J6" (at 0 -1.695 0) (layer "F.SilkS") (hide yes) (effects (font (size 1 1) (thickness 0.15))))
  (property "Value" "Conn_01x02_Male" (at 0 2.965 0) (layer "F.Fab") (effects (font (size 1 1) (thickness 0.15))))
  (fp_line (start 1.11 0.76) (end 1.11 1.965) (stroke (width 0.12) (type solid)) (layer "F.SilkS"))
  (fp_line (start 0.563471 0.76) (end 1.11 0.76) (stroke (width 0.12) (type solid)) (layer "F.SilkS"))
  (fp_line (start 0.30753 1.965) (end 1.11 1.965) (stroke (width 0.12) (type solid)) (layer "F.SilkS"))
  (fp_line (start -1.11 1.965) (end -0.30753 1.965) (stroke (width 0.12) (type solid)) (layer "F.SilkS"))
  (fp_line (start -1.11 0.76) (end -0.563471 0.76) (stroke (width 0.12) (type solid)) (layer "F.SilkS"))
  (fp_line (start -1.11 0.76) (end -1.11 1.965) (stroke (width 0.12) (type solid)) (layer "F.SilkS"))
  (fp_line (start -1.11 0) (end -1.11 -0.76) (stroke (width 0.12) (type solid)) (layer "F.SilkS"))
  (fp_line (start -1.11 -0.76) (end 0 -0.76) (stroke (width 0.12) (type solid)) (layer "F.SilkS"))
  (pad "1" thru_hole rect (at 0 0 180) (size 1 1) (drill 0.65) (layers "*.Cu" "*.Mask") (remove_unused_layers no) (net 1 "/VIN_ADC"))
  (pad "2" thru_hole oval (at 0 1.27 180) (size 1 1) (drill 0.65) (layers "*.Cu" "*.Mask") (remove_unused_layers no) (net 27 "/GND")))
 (gr_rect (start 100.0788 83.8282) (end 151.0788 105.8282) (stroke (width 0.1) (type solid)) (fill no) (layer "Edge.Cuts"))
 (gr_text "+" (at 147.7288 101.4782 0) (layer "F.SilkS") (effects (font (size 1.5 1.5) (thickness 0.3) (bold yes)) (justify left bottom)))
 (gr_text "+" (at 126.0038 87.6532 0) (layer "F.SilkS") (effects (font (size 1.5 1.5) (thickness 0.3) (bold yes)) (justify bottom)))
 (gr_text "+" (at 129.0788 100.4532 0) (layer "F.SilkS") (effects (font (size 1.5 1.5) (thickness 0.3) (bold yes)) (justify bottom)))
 (segment (start 105.0288 92.8282) (end 105.5373 92.8282) (width 0.2) (layer "F.Cu") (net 3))
 (segment (start 105.5373 92.8282) (end 108.2358 90.1297) (width 0.2) (layer "F.Cu") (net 3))
 (segment (start 107.7473 88.8597) (end 108.2358 88.8597) (width 0.2) (layer "F.Cu") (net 2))
 (segment (start 105.0288 91.5782) (end 107.7473 88.8597) (width 0.2) (layer "F.Cu") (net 2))
 (segment (start 106.2543 96.9282) (end 105.0788 96.9282) (width 0.2) (layer "F.Cu") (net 16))
 (segment (start 108.2358 98.9097) (end 106.2543 96.9282) (width 0.2) (layer "F.Cu") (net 16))
 (segment (start 107.0803 100.1797) (end 105.0788 98.1782) (width 0.2) (layer "F.Cu") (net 17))
 (segment (start 108.2358 100.1797) (end 107.0803 100.1797) (width 0.2) (layer "F.Cu") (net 17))
 (segment (start 120.5858 90.3697) (end 122.9163 90.3697) (width 0.2) (layer "F.Cu") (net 6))
 (segment (start 122.9163 90.3697) (end 123.9712 91.4246) (width 0.2) (layer "F.Cu") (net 6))
 (segment (start 120.5858 89.0997) (end 122.9163 89.0997) (width 0.2) (layer "F.Cu") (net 5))
 (segment (start 122.9163 89.0997) (end 123.9712 90.1546) (width 0.2) (layer "F.Cu") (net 5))
 (segment (start 148.6788 86.1782) (end 148.6788 94.0582) (width 0.4) (layer "F.Cu") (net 27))
 (segment (start 148.9038 85.9532) (end 148.6788 86.1782) (width 0.4) (layer "F.Cu") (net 27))
 (segment (start 140.8102 87.104393) (end 140.8102 99.0176) (width 0.4) (layer "B.Cu") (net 27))
 (segment (start 148.9038 85.9532) (end 147.6278 84.6772) (width 0.4) (layer "B.Cu") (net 27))
 (segment (start 143.237393 84.6772) (end 140.8102 87.104393) (width 0.4) (layer "B.Cu") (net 27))
 (segment (start 147.6278 84.6772) (end 143.237393 84.6772) (width 0.4) (layer "B.Cu") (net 27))
 (segment (start 140.8102 99.0176) (end 141.7112 99.9186) (width 0.4) (layer "B.Cu") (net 27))
 (segment (start 120.5858 87.8297) (end 120.581593 87.8297) (width 0.4) (layer "F.Cu") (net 4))
 (segment (start 120.581593 87.8297) (end 119.6848 88.726493) (width 0.4) (layer "F.Cu") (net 4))
 (segment (start 121.3089 87.1066) (end 120.5858 87.8297) (width 0.4) (layer "F.Cu") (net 4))
 (segment (start 119.6848 88.726493) (end 119.6848 96.9787) (width 0.4) (layer "F.Cu") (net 4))
 (segment (start 124.0982 87.1066) (end 121.3089 87.1066) (width 0.4) (layer "F.Cu") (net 4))
 (segment (start 119.6848 96.9787) (end 120.5858 97.8797) (width 0.4) (layer "F.Cu") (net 4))
 (segment (start 123.6953 101.6897) (end 124.2252 102.2196) (width 0.25) (layer "F.Cu") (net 7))
 (segment (start 120.212593 101.3207) (end 119.6848 100.792907) (width 0.4) (layer "B.Cu") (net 7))
 (segment (start 124.2252 102.2196) (end 121.1157 102.2196) (width 0.4) (layer "B.Cu") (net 7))
 (segment (start 121.1157 102.2196) (end 120.5858 101.6897) (width 0.4) (layer "B.Cu") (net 7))
 (segment (start 119.6848 92.5407) (end 120.5858 91.6397) (width 0.4) (layer "B.Cu") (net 7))
 (segment (start 120.2168 101.3207) (end 120.212593 101.3207) (width 0.4) (layer "B.Cu") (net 7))
 (segment (start 120.5858 101.6897) (end 120.2168 101.3207) (width 0.4) (layer "B.Cu") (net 7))
 (segment (start 119.6848 100.792907) (end 119.6848 92.5407) (width 0.4) (layer "B.Cu") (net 7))
 (segment (start 141.7112 87.4776) (end 143.7294 87.4776) (width 0.25) (layer "F.Cu") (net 8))
 (segment (start 143.7294 87.4776) (end 145.2788 85.9282) (width 0.25) (layer "F.Cu") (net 8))
 (segment (start 144.9994 88.7476) (end 145.2788 88.4682) (width 0.25) (layer "F.Cu") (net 9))
 (segment (start 141.7112 88.7476) (end 144.9994 88.7476) (width 0.25) (layer "F.Cu") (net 9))
 (segment (start 144.2882 90.0176) (end 145.2788 91.0082) (width 0.25) (layer "F.Cu") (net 10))
 (segment (start 141.7112 90.0176) (end 144.2882 90.0176) (width 0.25) (layer "F.Cu") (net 10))
 (segment (start 141.7112 94.9706) (end 144.1612 94.9706) (width 0.25) (layer "F.Cu") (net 12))
 (segment (start 144.1612 94.9706) (end 145.2788 96.0882) (width 0.25) (layer "F.Cu") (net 12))
 (segment (start 142.7592 101.1886) (end 145.2788 103.7082) (width 0.25) (layer "F.Cu") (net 15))
 (segment (start 141.7112 101.1886) (end 142.7592 101.1886) (width 0.25) (layer "F.Cu") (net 15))
 (segment (start 147.6228 104.9592) (end 144.2118 104.9592) (width 0.4) (layer "F.Cu") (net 1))
 (segment (start 148.7288 95.3782) (end 148.6788 95.3282) (width 0.4) (layer "F.Cu") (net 1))
 (segment (start 149.0538 103.4032) (end 148.7288 103.0782) (width 0.4) (layer "F.Cu") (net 1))
 (segment (start 149.0538 103.5282) (end 149.0538 103.4032) (width 0.4) (layer "F.Cu") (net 1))
 (segment (start 149.0538 103.5282) (end 147.6228 104.9592) (width 0.4) (layer "F.Cu") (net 1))
 (segment (start 148.7288 103.0782) (end 148.7288 95.3782) (width 0.4) (layer "F.Cu") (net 1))
 (segment (start 144.2118 104.9592) (end 141.7112 102.4586) (width 0.4) (layer "F.Cu") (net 1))
 (segment (start 120.9178 99.1497) (end 122.2028 97.8647) (width 0.2) (layer "F.Cu") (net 18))
 (segment (start 122.2028 97.8647) (end 122.2028 94.463) (width 0.2) (layer "F.Cu") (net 18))
 (segment (start 120.5858 99.1497) (end 120.9178 99.1497) (width 0.2) (layer "F.Cu") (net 18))
 (segment (start 122.2028 94.463) (end 123.9712 92.6946) (width 0.2) (layer "F.Cu") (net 18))
 (segment (start 120.5858 100.4197) (end 122.6038 98.4017) (width 0.2) (layer "F.Cu") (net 19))
 (segment (start 122.6038 98.4017) (end 122.6038 95.332) (width 0.2) (layer "F.Cu") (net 19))
 (segment (start 122.6038 95.332) (end 123.9712 93.9646) (width 0.2) (layer "F.Cu") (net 19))
 (segment (start 141.7112 93.7006) (end 145.1264 93.7006) (width 0.25) (layer "F.Cu") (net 11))
 (segment (start 145.1264 93.7006) (end 145.2788 93.5482) (width 0.25) (layer "F.Cu") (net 11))
 (segment (start 142.8912 96.2406) (end 145.2788 98.6282) (width 0.25) (layer "F.Cu") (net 13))
 (segment (start 141.7112 96.2406) (end 142.8912 96.2406) (width 0.25) (layer "F.Cu") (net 13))
 (segment (start 141.7112 97.6006) (end 145.2788 101.1682) (width 0.25) (layer "F.Cu") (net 14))
 (segment (start 141.7112 97.5106) (end 141.7112 97.6006) (width 0.25) (layer "F.Cu") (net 14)))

